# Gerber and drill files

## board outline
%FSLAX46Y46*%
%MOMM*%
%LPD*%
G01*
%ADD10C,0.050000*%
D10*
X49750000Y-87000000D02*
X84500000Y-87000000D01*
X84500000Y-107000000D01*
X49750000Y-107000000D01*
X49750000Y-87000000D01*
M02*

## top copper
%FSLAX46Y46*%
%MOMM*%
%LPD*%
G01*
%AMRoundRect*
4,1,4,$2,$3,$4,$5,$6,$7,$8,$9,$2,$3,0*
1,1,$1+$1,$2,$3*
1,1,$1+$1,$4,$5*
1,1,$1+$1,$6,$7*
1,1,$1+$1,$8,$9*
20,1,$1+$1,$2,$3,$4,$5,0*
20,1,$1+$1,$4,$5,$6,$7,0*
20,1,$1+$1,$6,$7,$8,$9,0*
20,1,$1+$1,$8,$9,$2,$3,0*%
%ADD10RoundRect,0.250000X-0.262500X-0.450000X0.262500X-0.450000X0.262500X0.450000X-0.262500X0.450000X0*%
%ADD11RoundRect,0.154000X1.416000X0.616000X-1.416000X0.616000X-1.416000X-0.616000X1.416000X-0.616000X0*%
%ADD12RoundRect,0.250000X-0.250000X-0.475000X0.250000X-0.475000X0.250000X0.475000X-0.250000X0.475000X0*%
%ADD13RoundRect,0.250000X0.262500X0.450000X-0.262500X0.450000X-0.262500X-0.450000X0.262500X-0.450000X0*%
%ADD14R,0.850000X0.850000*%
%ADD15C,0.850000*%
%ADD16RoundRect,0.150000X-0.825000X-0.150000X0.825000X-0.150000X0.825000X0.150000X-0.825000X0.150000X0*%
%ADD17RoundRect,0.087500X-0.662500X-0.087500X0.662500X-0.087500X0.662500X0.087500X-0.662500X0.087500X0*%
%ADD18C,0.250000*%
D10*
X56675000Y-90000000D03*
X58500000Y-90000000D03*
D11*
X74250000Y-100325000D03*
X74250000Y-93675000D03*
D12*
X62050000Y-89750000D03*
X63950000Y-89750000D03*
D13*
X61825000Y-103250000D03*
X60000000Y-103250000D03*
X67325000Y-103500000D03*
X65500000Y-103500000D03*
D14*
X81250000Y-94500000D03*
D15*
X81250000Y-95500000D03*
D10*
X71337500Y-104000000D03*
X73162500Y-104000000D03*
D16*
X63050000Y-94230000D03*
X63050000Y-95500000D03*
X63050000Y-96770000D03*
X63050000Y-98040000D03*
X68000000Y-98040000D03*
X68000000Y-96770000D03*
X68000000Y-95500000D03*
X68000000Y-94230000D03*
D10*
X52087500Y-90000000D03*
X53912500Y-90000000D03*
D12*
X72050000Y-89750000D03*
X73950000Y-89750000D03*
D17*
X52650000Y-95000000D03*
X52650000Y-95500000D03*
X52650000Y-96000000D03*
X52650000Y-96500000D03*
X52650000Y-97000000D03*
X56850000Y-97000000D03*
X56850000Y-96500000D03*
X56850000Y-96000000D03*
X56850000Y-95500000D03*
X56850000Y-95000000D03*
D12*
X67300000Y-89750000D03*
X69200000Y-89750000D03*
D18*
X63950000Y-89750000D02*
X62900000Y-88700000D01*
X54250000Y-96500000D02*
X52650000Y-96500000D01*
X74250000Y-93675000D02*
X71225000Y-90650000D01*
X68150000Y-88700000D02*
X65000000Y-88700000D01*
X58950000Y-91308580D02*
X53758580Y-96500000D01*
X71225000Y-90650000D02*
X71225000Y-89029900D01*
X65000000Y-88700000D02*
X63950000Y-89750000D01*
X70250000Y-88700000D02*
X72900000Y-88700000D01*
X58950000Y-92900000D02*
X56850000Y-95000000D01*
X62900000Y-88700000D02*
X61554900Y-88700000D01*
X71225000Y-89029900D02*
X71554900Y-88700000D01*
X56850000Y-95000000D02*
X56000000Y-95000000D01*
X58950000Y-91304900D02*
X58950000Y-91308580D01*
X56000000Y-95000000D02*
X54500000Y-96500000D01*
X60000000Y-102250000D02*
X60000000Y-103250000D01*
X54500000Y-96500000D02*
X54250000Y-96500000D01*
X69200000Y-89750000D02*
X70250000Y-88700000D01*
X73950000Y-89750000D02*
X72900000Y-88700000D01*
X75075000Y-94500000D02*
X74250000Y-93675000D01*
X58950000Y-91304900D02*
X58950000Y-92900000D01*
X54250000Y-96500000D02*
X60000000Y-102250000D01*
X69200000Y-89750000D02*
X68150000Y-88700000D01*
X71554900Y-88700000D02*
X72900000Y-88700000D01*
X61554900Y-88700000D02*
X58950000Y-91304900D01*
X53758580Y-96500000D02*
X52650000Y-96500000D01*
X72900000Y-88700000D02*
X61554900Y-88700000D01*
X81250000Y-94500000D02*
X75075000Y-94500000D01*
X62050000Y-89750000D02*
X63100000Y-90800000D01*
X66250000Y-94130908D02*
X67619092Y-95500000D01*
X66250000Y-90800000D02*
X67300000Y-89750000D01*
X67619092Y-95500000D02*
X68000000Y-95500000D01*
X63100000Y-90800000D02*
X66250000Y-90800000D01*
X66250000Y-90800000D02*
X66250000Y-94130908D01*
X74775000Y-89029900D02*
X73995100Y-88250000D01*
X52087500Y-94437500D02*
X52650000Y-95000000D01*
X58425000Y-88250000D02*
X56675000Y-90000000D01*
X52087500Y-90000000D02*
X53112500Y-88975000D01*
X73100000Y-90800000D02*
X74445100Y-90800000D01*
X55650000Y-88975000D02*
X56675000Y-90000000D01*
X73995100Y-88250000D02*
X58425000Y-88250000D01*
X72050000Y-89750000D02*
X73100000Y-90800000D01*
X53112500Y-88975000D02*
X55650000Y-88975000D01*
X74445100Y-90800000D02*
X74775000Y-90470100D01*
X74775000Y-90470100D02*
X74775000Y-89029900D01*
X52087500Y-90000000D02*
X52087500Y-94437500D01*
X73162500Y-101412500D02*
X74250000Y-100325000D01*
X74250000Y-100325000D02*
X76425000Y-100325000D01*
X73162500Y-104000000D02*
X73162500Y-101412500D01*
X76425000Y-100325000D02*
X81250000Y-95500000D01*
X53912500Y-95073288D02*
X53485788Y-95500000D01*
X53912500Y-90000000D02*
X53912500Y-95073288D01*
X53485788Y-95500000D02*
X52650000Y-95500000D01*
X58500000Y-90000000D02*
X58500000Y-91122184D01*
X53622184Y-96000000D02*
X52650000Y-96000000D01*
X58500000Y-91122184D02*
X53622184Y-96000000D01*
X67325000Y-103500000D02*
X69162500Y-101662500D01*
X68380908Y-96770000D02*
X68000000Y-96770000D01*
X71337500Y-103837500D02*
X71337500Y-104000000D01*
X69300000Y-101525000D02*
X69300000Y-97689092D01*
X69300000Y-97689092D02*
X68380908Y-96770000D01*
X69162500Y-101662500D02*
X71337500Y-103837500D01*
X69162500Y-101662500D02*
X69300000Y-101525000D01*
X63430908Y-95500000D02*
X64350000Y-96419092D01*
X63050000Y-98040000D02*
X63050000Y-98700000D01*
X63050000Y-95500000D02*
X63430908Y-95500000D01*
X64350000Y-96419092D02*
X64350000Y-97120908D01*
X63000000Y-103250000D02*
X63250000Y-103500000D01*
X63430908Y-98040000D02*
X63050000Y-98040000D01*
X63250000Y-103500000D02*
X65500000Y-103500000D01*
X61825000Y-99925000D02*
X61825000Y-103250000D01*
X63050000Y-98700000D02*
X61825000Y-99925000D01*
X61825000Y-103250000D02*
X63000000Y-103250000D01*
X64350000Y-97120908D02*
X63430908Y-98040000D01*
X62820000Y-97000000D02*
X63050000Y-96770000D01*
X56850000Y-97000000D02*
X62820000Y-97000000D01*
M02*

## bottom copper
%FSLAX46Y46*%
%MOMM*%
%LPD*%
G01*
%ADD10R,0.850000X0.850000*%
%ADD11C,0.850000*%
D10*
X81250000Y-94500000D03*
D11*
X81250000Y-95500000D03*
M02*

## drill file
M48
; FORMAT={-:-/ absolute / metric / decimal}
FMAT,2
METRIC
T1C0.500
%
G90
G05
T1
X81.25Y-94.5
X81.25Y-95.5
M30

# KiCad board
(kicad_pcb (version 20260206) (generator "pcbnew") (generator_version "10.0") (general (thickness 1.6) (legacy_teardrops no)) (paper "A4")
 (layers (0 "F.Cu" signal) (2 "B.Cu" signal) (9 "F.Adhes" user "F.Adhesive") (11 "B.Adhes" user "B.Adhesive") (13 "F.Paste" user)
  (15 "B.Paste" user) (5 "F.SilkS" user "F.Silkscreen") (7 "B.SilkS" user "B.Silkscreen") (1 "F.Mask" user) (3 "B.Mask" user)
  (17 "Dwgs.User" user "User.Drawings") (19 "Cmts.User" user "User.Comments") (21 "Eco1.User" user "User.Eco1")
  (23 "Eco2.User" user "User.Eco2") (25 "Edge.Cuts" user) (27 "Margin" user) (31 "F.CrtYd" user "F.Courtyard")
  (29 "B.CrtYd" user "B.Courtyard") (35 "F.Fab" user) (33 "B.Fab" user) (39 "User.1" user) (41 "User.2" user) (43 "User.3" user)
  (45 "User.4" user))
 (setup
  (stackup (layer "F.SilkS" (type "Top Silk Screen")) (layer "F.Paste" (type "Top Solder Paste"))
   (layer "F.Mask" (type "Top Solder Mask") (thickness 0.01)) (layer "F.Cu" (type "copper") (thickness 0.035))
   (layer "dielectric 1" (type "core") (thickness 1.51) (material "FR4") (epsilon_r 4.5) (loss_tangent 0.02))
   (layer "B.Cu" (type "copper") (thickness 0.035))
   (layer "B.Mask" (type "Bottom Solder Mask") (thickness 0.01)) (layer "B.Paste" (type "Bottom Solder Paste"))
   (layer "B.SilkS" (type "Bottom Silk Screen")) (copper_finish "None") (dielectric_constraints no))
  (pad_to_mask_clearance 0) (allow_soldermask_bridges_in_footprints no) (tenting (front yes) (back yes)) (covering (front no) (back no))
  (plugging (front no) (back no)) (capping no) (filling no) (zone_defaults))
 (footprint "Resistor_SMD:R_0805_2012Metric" (layer "F.Cu") (at 57.5875 90)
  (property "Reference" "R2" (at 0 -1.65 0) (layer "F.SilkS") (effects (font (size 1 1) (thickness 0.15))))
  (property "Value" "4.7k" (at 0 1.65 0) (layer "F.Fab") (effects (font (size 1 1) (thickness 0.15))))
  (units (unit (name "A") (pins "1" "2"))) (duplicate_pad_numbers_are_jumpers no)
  (pad "1" smd roundrect (at -0.9125 0) (size 1.025 1.4) (layers "F.Cu" "F.Mask" "F.Paste") (roundrect_rratio 0.243902) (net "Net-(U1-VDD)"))
  (pad "2" smd roundrect (at 0.9125 0) (size 1.025 1.4) (layers "F.Cu" "F.Mask" "F.Paste") (roundrect_rratio 0.243902) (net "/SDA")))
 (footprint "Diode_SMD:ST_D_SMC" (layer "F.Cu") (at 74.25 97 90)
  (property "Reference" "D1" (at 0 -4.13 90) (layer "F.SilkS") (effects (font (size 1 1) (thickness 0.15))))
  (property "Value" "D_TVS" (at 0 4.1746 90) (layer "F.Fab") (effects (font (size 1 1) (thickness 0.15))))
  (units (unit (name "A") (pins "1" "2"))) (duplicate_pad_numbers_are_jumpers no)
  (pad "1" smd roundrect (at -3.325 0 180) (size 3.14 1.54) (layers "F.Cu" "F.Mask" "F.Paste") (roundrect_rratio 0.1) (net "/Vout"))
  (pad "2" smd roundrect (at 3.325 0 180) (size 3.14 1.54) (layers "F.Cu" "F.Mask" "F.Paste") (roundrect_rratio 0.1) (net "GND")))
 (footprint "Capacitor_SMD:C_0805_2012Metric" (layer "F.Cu") (at 63 89.75)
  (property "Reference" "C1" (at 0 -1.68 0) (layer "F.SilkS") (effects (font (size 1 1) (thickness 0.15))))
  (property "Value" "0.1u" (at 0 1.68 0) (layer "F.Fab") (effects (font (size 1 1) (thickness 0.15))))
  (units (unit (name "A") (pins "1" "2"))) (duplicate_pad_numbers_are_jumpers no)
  (pad "1" smd roundrect (at -0.95 0) (size 1 1.45) (layers "F.Cu" "F.Mask" "F.Paste") (roundrect_rratio 0.25) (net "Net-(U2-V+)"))
  (pad "2" smd roundrect (at 0.95 0) (size 1 1.45) (layers "F.Cu" "F.Mask" "F.Paste") (roundrect_rratio 0.25) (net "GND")))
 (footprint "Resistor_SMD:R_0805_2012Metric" (layer "F.Cu") (at 60.9125 103.25 180)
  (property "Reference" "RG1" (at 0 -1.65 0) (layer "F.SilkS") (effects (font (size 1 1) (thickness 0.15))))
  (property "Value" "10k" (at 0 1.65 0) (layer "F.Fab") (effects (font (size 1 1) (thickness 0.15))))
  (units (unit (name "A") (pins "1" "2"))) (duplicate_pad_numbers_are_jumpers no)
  (pad "1" smd roundrect (at -0.9125 0 180) (size 1.025 1.4) (layers "F.Cu" "F.Mask" "F.Paste") (roundrect_rratio 0.243902)
   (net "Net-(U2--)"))
  (pad "2" smd roundrect (at 0.9125 0 180) (size 1.025 1.4) (layers "F.Cu" "F.Mask" "F.Paste") (roundrect_rratio 0.243902) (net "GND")))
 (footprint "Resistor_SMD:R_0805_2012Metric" (layer "F.Cu") (at 66.4125 103.5 180)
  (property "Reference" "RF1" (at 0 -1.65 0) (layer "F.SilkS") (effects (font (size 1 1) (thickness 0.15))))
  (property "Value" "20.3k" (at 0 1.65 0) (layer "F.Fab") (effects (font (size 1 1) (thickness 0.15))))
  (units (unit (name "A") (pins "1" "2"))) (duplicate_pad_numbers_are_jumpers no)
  (pad "1" smd roundrect (at -0.9125 0 180) (size 1.025 1.4) (layers "F.Cu" "F.Mask" "F.Paste") (roundrect_rratio 0.243902)
   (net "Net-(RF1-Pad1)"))
  (pad "2" smd roundrect (at 0.9125 0 180) (size 1.025 1.4) (layers "F.Cu" "F.Mask" "F.Paste") (roundrect_rratio 0.243902)
   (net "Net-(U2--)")))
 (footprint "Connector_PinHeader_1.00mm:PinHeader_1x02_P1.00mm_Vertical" (layer "F.Cu") (at 81.25 94.5)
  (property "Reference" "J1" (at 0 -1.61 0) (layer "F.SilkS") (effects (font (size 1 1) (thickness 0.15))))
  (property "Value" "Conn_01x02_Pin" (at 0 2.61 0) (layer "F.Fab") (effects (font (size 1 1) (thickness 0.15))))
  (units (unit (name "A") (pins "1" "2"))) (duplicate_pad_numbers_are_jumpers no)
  (pad "1" thru_hole rect (at 0 0) (size 0.85 0.85) (drill 0.5) (layers "*.Cu" "*.Mask") (remove_unused_layers no) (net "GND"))
  (pad "2" thru_hole circle (at 0 1) (size 0.85 0.85) (drill 0.5) (layers "*.Cu" "*.Mask") (remove_unused_layers no) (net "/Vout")))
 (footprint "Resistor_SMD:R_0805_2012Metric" (layer "F.Cu") (at 72.25 104)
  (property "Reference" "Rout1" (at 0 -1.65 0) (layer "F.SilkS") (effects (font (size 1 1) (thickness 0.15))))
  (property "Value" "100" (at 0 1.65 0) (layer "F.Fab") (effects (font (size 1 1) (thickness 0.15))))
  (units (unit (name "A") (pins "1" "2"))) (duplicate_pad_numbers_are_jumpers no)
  (pad "1" smd roundrect (at -0.9125 0) (size 1.025 1.4) (layers "F.Cu" "F.Mask" "F.Paste") (roundrect_rratio 0.243902)
   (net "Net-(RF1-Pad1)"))
  (pad "2" smd roundrect (at 0.9125 0) (size 1.025 1.4) (layers "F.Cu" "F.Mask" "F.Paste") (roundrect_rratio 0.243902) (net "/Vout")))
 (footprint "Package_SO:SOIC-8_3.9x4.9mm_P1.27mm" (layer "F.Cu") (at 65.525 96.135)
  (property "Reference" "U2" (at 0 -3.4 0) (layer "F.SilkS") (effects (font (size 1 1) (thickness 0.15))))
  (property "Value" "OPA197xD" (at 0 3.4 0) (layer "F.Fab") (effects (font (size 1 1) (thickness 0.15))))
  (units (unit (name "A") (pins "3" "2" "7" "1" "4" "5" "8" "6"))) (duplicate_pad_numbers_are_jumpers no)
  (pad "1" smd roundrect (at -2.475 -1.905) (size 1.95 0.6) (layers "F.Cu" "F.Mask" "F.Paste") (roundrect_rratio 0.25)
   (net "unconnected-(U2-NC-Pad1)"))
  (pad "2" smd roundrect (at -2.475 -0.635) (size 1.95 0.6) (layers "F.Cu" "F.Mask" "F.Paste") (roundrect_rratio 0.25) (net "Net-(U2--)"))
  (pad "3" smd roundrect (at -2.475 0.635) (size 1.95 0.6) (layers "F.Cu" "F.Mask" "F.Paste") (roundrect_rratio 0.25) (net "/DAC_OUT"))
  (pad "4" smd roundrect (at -2.475 1.905) (size 1.95 0.6) (layers "F.Cu" "F.Mask" "F.Paste") (roundrect_rratio 0.25) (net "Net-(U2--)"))
  (pad "5" smd roundrect (at 2.475 1.905) (size 1.95 0.6) (layers "F.Cu" "F.Mask" "F.Paste") (roundrect_rratio 0.25)
   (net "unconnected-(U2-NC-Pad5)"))
  (pad "6" smd roundrect (at 2.475 0.635) (size 1.95 0.6) (layers "F.Cu" "F.Mask" "F.Paste") (roundrect_rratio 0.25) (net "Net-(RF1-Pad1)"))
  (pad "7" smd roundrect (at 2.475 -0.635) (size 1.95 0.6) (layers "F.Cu" "F.Mask" "F.Paste") (roundrect_rratio 0.25) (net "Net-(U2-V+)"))
  (pad "8" smd roundrect (at 2.475 -1.905) (size 1.95 0.6) (layers "F.Cu" "F.Mask" "F.Paste") (roundrect_rratio 0.25)
   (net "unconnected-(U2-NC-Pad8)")))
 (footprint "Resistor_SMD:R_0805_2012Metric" (layer "F.Cu") (at 53 90)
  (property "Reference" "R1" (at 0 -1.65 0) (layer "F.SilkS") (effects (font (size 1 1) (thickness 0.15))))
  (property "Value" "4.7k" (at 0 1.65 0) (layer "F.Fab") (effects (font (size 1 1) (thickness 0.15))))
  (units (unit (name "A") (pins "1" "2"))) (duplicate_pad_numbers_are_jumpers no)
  (pad "1" smd roundrect (at -0.9125 0) (size 1.025 1.4) (layers "F.Cu" "F.Mask" "F.Paste") (roundrect_rratio 0.243902) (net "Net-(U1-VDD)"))
  (pad "2" smd roundrect (at 0.9125 0) (size 1.025 1.4) (layers "F.Cu" "F.Mask" "F.Paste") (roundrect_rratio 0.243902) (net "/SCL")))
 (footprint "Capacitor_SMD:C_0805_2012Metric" (layer "F.Cu") (at 73 89.75)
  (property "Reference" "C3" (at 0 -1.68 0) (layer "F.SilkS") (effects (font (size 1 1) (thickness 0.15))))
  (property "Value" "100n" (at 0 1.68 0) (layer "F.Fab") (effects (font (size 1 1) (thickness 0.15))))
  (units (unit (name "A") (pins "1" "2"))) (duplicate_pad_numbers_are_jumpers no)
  (pad "1" smd roundrect (at -0.95 0) (size 1 1.45) (layers "F.Cu" "F.Mask" "F.Paste") (roundrect_rratio 0.25) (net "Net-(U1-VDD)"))
  (pad "2" smd roundrect (at 0.95 0) (size 1 1.45) (layers "F.Cu" "F.Mask" "F.Paste") (roundrect_rratio 0.25) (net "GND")))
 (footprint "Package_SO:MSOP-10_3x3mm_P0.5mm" (layer "F.Cu") (at 54.75 96)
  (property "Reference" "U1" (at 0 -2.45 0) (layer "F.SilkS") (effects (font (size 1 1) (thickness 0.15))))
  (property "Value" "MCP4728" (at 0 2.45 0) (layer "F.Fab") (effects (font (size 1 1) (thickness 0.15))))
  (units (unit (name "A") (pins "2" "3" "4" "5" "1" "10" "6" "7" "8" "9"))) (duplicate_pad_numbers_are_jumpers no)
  (pad "1" smd roundrect (at -2.1 -1) (size 1.5 0.35) (layers "F.Cu" "F.Mask" "F.Paste") (roundrect_rratio 0.25) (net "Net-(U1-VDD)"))
  (pad "2" smd roundrect (at -2.1 -0.5) (size 1.5 0.35) (layers "F.Cu" "F.Mask" "F.Paste") (roundrect_rratio 0.25) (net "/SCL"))
  (pad "3" smd roundrect (at -2.1 0) (size 1.5 0.35) (layers "F.Cu" "F.Mask" "F.Paste") (roundrect_rratio 0.25) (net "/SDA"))
  (pad "4" smd roundrect (at -2.1 0.5) (size 1.5 0.35) (layers "F.Cu" "F.Mask" "F.Paste") (roundrect_rratio 0.25) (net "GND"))
  (pad "5" smd roundrect (at -2.1 1) (size 1.5 0.35) (layers "F.Cu" "F.Mask" "F.Paste") (roundrect_rratio 0.25)
   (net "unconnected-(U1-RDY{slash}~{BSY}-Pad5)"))
  (pad "6" smd roundrect (at 2.1 1) (size 1.5 0.35) (layers "F.Cu" "F.Mask" "F.Paste") (roundrect_rratio 0.25) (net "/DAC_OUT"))
  (pad "7" smd roundrect (at 2.1 0.5) (size 1.5 0.35) (layers "F.Cu" "F.Mask" "F.Paste") (roundrect_rratio 0.25)
   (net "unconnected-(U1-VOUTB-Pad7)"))
  (pad "8" smd roundrect (at 2.1 0) (size 1.5 0.35) (layers "F.Cu" "F.Mask" "F.Paste") (roundrect_rratio 0.25)
   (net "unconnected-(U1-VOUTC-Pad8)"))
  (pad "9" smd roundrect (at 2.1 -0.5) (size 1.5 0.35) (layers "F.Cu" "F.Mask" "F.Paste") (roundrect_rratio 0.25)
   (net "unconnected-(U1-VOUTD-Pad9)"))
  (pad "10" smd roundrect (at 2.1 -1) (size 1.5 0.35) (layers "F.Cu" "F.Mask" "F.Paste") (roundrect_rratio 0.25) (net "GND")))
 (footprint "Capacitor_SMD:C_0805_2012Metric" (layer "F.Cu") (at 68.25 89.75)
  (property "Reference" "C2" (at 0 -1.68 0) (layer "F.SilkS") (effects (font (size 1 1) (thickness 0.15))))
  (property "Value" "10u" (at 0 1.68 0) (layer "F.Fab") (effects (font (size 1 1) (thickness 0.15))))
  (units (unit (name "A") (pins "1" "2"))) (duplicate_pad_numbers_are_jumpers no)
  (pad "1" smd roundrect (at -0.95 0) (size 1 1.45) (layers "F.Cu" "F.Mask" "F.Paste") (roundrect_rratio 0.25) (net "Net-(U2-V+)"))
  (pad "2" smd roundrect (at 0.95 0) (size 1 1.45) (layers "F.Cu" "F.Mask" "F.Paste") (roundrect_rratio 0.25) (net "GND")))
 (gr_rect (start 49.75 87) (end 84.5 107) (stroke (width 0.05) (type default)) (fill no) (locked yes) (layer "Edge.Cuts"))
 (segment (start 63.95 89.75) (end 62.9 88.7) (width 0.25) (layer "F.Cu") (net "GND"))
 (segment (start 54.25 96.5) (end 52.65 96.5) (width 0.25) (layer "F.Cu") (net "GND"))
 (segment (start 74.25 93.675) (end 71.225 90.65) (width 0.25) (layer "F.Cu") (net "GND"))
 (segment (start 68.15 88.7) (end 65 88.7) (width 0.25) (layer "F.Cu") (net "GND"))
 (segment (start 58.95 91.30858) (end 53.75858 96.5) (width 0.25) (layer "F.Cu") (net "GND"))
 (segment (start 71.225 90.65) (end 71.225 89.0299) (width 0.25) (layer "F.Cu") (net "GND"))
 (segment (start 65 88.7) (end 63.95 89.75) (width 0.25) (layer "F.Cu") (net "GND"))
 (segment (start 70.25 88.7) (end 72.9 88.7) (width 0.25) (layer "F.Cu") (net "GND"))
 (segment (start 58.95 92.9) (end 56.85 95) (width 0.25) (layer "F.Cu") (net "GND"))
 (segment (start 62.9 88.7) (end 61.5549 88.7) (width 0.25) (layer "F.Cu") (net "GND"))
 (segment (start 71.225 89.0299) (end 71.5549 88.7) (width 0.25) (layer "F.Cu") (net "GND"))
 (segment (start 56.85 95) (end 56 95) (width 0.25) (layer "F.Cu") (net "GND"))
 (segment (start 58.95 91.3049) (end 58.95 91.30858) (width 0.25) (layer "F.Cu") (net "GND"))
 (segment (start 56 95) (end 54.5 96.5) (width 0.25) (layer "F.Cu") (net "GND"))
 (segment (start 60 102.25) (end 60 103.25) (width 0.25) (layer "F.Cu") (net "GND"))
 (segment (start 54.5 96.5) (end 54.25 96.5) (width 0.25) (layer "F.Cu") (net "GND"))
 (segment (start 69.2 89.75) (end 70.25 88.7) (width 0.25) (layer "F.Cu") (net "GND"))
 (segment (start 73.95 89.75) (end 72.9 88.7) (width 0.25) (layer "F.Cu") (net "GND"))
 (segment (start 75.075 94.5) (end 74.25 93.675) (width 0.25) (layer "F.Cu") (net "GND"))
 (segment (start 58.95 91.3049) (end 58.95 92.9) (width 0.25) (layer "F.Cu") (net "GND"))
 (segment (start 54.25 96.5) (end 60 102.25) (width 0.25) (layer "F.Cu") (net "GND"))
 (segment (start 69.2 89.75) (end 68.15 88.7) (width 0.25) (layer "F.Cu") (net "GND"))
 (segment (start 71.5549 88.7) (end 72.9 88.7) (width 0.25) (layer "F.Cu") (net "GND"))
 (segment (start 61.5549 88.7) (end 58.95 91.3049) (width 0.25) (layer "F.Cu") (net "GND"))
 (segment (start 53.75858 96.5) (end 52.65 96.5) (width 0.25) (layer "F.Cu") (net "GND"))
 (segment (start 72.9 88.7) (end 61.5549 88.7) (width 0.25) (layer "F.Cu") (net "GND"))
 (segment (start 81.25 94.5) (end 75.075 94.5) (width 0.25) (layer "F.Cu") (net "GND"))
 (segment (start 62.05 89.75) (end 63.1 90.8) (width 0.25) (layer "F.Cu") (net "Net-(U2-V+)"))
 (segment (start 66.25 94.130908) (end 67.619092 95.5) (width 0.25) (layer "F.Cu") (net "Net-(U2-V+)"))
 (segment (start 66.25 90.8) (end 67.3 89.75) (width 0.25) (layer "F.Cu") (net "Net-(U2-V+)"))
 (segment (start 67.619092 95.5) (end 68 95.5) (width 0.25) (layer "F.Cu") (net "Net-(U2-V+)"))
 (segment (start 63.1 90.8) (end 66.25 90.8) (width 0.25) (layer "F.Cu") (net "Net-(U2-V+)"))
 (segment (start 66.25 90.8) (end 66.25 94.130908) (width 0.25) (layer "F.Cu") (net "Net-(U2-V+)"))
 (segment (start 74.775 89.0299) (end 73.9951 88.25) (width 0.25) (layer "F.Cu") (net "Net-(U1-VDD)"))
 (segment (start 52.0875 94.4375) (end 52.65 95) (width 0.25) (layer "F.Cu") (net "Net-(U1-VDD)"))
 (segment (start 58.425 88.25) (end 56.675 90) (width 0.25) (layer "F.Cu") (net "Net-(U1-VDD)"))
 (segment (start 52.0875 90) (end 53.1125 88.975) (width 0.25) (layer "F.Cu") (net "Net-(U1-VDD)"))
 (segment (start 73.1 90.8) (end 74.4451 90.8) (width 0.25) (layer "F.Cu") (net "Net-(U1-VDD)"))
 (segment (start 55.65 88.975) (end 56.675 90) (width 0.25) (layer "F.Cu") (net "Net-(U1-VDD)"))
 (segment (start 73.9951 88.25) (end 58.425 88.25) (width 0.25) (layer "F.Cu") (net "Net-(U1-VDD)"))
 (segment (start 72.05 89.75) (end 73.1 90.8) (width 0.25) (layer "F.Cu") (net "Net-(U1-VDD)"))
 (segment (start 53.1125 88.975) (end 55.65 88.975) (width 0.25) (layer "F.Cu") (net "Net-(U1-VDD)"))
 (segment (start 74.4451 90.8) (end 74.775 90.4701) (width 0.25) (layer "F.Cu") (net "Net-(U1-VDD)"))
 (segment (start 74.775 90.4701) (end 74.775 89.0299) (width 0.25) (layer "F.Cu") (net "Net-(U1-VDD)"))
 (segment (start 52.0875 90) (end 52.0875 94.4375) (width 0.25) (layer "F.Cu") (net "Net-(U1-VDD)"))
 (segment (start 73.1625 101.4125) (end 74.25 100.325) (width 0.25) (layer "F.Cu") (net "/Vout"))
 (segment (start 74.25 100.325) (end 76.425 100.325) (width 0.25) (layer "F.Cu") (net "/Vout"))
 (segment (start 73.1625 104) (end 73.1625 101.4125) (width 0.25) (layer "F.Cu") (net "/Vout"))
 (segment (start 76.425 100.325) (end 81.25 95.5) (width 0.25) (layer "F.Cu") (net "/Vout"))
 (segment (start 53.9125 95.073288) (end 53.485788 95.5) (width 0.25) (layer "F.Cu") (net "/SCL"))
 (segment (start 53.9125 90) (end 53.9125 95.073288) (width 0.25) (layer "F.Cu") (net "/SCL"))
 (segment (start 53.485788 95.5) (end 52.65 95.5) (width 0.25) (layer "F.Cu") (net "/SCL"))
 (segment (start 58.5 90) (end 58.5 91.122184) (width 0.25) (layer "F.Cu") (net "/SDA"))
 (segment (start 53.622184 96) (end 52.65 96) (width 0.25) (layer "F.Cu") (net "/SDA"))
 (segment (start 58.5 91.122184) (end 53.622184 96) (width 0.25) (layer "F.Cu") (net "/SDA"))
 (segment (start 67.325 103.5) (end 69.1625 101.6625) (width 0.25) (layer "F.Cu") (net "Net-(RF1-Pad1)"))
 (segment (start 68.380908 96.77) (end 68 96.77) (width 0.25) (layer "F.Cu") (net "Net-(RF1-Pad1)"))
 (segment (start 71.3375 103.8375) (end 71.3375 104) (width 0.25) (layer "F.Cu") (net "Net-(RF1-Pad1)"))
 (segment (start 69.3 101.525) (end 69.3 97.689092) (width 0.25) (layer "F.Cu") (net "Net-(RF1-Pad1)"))
 (segment (start 69.3 97.689092) (end 68.380908 96.77) (width 0.25) (layer "F.Cu") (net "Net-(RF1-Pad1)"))
 (segment (start 69.1625 101.6625) (end 71.3375 103.8375) (width 0.25) (layer "F.Cu") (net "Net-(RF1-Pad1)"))
 (segment (start 69.1625 101.6625) (end 69.3 101.525) (width 0.25) (layer "F.Cu") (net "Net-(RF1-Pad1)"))
 (segment (start 63.430908 95.5) (end 64.35 96.419092) (width 0.25) (layer "F.Cu") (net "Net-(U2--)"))
 (segment (start 63.05 98.04) (end 63.05 98.7) (width 0.25) (layer "F.Cu") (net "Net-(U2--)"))
 (segment (start 63.05 95.5) (end 63.430908 95.5) (width 0.25) (layer "F.Cu") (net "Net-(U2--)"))
 (segment (start 64.35 96.419092) (end 64.35 97.120908) (width 0.25) (layer "F.Cu") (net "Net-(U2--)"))
 (segment (start 63 103.25) (end 63.25 103.5) (width 0.25) (layer "F.Cu") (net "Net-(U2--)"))
 (segment (start 63.430908 98.04) (end 63.05 98.04) (width 0.25) (layer "F.Cu") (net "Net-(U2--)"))
 (segment (start 63.25 103.5) (end 65.5 103.5) (width 0.25) (layer "F.Cu") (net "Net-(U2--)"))
 (segment (start 61.825 99.925) (end 61.825 103.25) (width 0.25) (layer "F.Cu") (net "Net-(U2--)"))
 (segment (start 63.05 98.7) (end 61.825 99.925) (width 0.25) (layer "F.Cu") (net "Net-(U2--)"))
 (segment (start 61.825 103.25) (end 63 103.25) (width 0.25) (layer "F.Cu") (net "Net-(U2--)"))
 (segment (start 64.35 97.120908) (end 63.430908 98.04) (width 0.25) (layer "F.Cu") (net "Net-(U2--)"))
 (segment (start 62.82 97) (end 63.05 96.77) (width 0.25) (layer "F.Cu") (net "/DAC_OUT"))
 (segment (start 56.85 97) (end 62.82 97) (width 0.25) (layer "F.Cu") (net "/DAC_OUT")))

